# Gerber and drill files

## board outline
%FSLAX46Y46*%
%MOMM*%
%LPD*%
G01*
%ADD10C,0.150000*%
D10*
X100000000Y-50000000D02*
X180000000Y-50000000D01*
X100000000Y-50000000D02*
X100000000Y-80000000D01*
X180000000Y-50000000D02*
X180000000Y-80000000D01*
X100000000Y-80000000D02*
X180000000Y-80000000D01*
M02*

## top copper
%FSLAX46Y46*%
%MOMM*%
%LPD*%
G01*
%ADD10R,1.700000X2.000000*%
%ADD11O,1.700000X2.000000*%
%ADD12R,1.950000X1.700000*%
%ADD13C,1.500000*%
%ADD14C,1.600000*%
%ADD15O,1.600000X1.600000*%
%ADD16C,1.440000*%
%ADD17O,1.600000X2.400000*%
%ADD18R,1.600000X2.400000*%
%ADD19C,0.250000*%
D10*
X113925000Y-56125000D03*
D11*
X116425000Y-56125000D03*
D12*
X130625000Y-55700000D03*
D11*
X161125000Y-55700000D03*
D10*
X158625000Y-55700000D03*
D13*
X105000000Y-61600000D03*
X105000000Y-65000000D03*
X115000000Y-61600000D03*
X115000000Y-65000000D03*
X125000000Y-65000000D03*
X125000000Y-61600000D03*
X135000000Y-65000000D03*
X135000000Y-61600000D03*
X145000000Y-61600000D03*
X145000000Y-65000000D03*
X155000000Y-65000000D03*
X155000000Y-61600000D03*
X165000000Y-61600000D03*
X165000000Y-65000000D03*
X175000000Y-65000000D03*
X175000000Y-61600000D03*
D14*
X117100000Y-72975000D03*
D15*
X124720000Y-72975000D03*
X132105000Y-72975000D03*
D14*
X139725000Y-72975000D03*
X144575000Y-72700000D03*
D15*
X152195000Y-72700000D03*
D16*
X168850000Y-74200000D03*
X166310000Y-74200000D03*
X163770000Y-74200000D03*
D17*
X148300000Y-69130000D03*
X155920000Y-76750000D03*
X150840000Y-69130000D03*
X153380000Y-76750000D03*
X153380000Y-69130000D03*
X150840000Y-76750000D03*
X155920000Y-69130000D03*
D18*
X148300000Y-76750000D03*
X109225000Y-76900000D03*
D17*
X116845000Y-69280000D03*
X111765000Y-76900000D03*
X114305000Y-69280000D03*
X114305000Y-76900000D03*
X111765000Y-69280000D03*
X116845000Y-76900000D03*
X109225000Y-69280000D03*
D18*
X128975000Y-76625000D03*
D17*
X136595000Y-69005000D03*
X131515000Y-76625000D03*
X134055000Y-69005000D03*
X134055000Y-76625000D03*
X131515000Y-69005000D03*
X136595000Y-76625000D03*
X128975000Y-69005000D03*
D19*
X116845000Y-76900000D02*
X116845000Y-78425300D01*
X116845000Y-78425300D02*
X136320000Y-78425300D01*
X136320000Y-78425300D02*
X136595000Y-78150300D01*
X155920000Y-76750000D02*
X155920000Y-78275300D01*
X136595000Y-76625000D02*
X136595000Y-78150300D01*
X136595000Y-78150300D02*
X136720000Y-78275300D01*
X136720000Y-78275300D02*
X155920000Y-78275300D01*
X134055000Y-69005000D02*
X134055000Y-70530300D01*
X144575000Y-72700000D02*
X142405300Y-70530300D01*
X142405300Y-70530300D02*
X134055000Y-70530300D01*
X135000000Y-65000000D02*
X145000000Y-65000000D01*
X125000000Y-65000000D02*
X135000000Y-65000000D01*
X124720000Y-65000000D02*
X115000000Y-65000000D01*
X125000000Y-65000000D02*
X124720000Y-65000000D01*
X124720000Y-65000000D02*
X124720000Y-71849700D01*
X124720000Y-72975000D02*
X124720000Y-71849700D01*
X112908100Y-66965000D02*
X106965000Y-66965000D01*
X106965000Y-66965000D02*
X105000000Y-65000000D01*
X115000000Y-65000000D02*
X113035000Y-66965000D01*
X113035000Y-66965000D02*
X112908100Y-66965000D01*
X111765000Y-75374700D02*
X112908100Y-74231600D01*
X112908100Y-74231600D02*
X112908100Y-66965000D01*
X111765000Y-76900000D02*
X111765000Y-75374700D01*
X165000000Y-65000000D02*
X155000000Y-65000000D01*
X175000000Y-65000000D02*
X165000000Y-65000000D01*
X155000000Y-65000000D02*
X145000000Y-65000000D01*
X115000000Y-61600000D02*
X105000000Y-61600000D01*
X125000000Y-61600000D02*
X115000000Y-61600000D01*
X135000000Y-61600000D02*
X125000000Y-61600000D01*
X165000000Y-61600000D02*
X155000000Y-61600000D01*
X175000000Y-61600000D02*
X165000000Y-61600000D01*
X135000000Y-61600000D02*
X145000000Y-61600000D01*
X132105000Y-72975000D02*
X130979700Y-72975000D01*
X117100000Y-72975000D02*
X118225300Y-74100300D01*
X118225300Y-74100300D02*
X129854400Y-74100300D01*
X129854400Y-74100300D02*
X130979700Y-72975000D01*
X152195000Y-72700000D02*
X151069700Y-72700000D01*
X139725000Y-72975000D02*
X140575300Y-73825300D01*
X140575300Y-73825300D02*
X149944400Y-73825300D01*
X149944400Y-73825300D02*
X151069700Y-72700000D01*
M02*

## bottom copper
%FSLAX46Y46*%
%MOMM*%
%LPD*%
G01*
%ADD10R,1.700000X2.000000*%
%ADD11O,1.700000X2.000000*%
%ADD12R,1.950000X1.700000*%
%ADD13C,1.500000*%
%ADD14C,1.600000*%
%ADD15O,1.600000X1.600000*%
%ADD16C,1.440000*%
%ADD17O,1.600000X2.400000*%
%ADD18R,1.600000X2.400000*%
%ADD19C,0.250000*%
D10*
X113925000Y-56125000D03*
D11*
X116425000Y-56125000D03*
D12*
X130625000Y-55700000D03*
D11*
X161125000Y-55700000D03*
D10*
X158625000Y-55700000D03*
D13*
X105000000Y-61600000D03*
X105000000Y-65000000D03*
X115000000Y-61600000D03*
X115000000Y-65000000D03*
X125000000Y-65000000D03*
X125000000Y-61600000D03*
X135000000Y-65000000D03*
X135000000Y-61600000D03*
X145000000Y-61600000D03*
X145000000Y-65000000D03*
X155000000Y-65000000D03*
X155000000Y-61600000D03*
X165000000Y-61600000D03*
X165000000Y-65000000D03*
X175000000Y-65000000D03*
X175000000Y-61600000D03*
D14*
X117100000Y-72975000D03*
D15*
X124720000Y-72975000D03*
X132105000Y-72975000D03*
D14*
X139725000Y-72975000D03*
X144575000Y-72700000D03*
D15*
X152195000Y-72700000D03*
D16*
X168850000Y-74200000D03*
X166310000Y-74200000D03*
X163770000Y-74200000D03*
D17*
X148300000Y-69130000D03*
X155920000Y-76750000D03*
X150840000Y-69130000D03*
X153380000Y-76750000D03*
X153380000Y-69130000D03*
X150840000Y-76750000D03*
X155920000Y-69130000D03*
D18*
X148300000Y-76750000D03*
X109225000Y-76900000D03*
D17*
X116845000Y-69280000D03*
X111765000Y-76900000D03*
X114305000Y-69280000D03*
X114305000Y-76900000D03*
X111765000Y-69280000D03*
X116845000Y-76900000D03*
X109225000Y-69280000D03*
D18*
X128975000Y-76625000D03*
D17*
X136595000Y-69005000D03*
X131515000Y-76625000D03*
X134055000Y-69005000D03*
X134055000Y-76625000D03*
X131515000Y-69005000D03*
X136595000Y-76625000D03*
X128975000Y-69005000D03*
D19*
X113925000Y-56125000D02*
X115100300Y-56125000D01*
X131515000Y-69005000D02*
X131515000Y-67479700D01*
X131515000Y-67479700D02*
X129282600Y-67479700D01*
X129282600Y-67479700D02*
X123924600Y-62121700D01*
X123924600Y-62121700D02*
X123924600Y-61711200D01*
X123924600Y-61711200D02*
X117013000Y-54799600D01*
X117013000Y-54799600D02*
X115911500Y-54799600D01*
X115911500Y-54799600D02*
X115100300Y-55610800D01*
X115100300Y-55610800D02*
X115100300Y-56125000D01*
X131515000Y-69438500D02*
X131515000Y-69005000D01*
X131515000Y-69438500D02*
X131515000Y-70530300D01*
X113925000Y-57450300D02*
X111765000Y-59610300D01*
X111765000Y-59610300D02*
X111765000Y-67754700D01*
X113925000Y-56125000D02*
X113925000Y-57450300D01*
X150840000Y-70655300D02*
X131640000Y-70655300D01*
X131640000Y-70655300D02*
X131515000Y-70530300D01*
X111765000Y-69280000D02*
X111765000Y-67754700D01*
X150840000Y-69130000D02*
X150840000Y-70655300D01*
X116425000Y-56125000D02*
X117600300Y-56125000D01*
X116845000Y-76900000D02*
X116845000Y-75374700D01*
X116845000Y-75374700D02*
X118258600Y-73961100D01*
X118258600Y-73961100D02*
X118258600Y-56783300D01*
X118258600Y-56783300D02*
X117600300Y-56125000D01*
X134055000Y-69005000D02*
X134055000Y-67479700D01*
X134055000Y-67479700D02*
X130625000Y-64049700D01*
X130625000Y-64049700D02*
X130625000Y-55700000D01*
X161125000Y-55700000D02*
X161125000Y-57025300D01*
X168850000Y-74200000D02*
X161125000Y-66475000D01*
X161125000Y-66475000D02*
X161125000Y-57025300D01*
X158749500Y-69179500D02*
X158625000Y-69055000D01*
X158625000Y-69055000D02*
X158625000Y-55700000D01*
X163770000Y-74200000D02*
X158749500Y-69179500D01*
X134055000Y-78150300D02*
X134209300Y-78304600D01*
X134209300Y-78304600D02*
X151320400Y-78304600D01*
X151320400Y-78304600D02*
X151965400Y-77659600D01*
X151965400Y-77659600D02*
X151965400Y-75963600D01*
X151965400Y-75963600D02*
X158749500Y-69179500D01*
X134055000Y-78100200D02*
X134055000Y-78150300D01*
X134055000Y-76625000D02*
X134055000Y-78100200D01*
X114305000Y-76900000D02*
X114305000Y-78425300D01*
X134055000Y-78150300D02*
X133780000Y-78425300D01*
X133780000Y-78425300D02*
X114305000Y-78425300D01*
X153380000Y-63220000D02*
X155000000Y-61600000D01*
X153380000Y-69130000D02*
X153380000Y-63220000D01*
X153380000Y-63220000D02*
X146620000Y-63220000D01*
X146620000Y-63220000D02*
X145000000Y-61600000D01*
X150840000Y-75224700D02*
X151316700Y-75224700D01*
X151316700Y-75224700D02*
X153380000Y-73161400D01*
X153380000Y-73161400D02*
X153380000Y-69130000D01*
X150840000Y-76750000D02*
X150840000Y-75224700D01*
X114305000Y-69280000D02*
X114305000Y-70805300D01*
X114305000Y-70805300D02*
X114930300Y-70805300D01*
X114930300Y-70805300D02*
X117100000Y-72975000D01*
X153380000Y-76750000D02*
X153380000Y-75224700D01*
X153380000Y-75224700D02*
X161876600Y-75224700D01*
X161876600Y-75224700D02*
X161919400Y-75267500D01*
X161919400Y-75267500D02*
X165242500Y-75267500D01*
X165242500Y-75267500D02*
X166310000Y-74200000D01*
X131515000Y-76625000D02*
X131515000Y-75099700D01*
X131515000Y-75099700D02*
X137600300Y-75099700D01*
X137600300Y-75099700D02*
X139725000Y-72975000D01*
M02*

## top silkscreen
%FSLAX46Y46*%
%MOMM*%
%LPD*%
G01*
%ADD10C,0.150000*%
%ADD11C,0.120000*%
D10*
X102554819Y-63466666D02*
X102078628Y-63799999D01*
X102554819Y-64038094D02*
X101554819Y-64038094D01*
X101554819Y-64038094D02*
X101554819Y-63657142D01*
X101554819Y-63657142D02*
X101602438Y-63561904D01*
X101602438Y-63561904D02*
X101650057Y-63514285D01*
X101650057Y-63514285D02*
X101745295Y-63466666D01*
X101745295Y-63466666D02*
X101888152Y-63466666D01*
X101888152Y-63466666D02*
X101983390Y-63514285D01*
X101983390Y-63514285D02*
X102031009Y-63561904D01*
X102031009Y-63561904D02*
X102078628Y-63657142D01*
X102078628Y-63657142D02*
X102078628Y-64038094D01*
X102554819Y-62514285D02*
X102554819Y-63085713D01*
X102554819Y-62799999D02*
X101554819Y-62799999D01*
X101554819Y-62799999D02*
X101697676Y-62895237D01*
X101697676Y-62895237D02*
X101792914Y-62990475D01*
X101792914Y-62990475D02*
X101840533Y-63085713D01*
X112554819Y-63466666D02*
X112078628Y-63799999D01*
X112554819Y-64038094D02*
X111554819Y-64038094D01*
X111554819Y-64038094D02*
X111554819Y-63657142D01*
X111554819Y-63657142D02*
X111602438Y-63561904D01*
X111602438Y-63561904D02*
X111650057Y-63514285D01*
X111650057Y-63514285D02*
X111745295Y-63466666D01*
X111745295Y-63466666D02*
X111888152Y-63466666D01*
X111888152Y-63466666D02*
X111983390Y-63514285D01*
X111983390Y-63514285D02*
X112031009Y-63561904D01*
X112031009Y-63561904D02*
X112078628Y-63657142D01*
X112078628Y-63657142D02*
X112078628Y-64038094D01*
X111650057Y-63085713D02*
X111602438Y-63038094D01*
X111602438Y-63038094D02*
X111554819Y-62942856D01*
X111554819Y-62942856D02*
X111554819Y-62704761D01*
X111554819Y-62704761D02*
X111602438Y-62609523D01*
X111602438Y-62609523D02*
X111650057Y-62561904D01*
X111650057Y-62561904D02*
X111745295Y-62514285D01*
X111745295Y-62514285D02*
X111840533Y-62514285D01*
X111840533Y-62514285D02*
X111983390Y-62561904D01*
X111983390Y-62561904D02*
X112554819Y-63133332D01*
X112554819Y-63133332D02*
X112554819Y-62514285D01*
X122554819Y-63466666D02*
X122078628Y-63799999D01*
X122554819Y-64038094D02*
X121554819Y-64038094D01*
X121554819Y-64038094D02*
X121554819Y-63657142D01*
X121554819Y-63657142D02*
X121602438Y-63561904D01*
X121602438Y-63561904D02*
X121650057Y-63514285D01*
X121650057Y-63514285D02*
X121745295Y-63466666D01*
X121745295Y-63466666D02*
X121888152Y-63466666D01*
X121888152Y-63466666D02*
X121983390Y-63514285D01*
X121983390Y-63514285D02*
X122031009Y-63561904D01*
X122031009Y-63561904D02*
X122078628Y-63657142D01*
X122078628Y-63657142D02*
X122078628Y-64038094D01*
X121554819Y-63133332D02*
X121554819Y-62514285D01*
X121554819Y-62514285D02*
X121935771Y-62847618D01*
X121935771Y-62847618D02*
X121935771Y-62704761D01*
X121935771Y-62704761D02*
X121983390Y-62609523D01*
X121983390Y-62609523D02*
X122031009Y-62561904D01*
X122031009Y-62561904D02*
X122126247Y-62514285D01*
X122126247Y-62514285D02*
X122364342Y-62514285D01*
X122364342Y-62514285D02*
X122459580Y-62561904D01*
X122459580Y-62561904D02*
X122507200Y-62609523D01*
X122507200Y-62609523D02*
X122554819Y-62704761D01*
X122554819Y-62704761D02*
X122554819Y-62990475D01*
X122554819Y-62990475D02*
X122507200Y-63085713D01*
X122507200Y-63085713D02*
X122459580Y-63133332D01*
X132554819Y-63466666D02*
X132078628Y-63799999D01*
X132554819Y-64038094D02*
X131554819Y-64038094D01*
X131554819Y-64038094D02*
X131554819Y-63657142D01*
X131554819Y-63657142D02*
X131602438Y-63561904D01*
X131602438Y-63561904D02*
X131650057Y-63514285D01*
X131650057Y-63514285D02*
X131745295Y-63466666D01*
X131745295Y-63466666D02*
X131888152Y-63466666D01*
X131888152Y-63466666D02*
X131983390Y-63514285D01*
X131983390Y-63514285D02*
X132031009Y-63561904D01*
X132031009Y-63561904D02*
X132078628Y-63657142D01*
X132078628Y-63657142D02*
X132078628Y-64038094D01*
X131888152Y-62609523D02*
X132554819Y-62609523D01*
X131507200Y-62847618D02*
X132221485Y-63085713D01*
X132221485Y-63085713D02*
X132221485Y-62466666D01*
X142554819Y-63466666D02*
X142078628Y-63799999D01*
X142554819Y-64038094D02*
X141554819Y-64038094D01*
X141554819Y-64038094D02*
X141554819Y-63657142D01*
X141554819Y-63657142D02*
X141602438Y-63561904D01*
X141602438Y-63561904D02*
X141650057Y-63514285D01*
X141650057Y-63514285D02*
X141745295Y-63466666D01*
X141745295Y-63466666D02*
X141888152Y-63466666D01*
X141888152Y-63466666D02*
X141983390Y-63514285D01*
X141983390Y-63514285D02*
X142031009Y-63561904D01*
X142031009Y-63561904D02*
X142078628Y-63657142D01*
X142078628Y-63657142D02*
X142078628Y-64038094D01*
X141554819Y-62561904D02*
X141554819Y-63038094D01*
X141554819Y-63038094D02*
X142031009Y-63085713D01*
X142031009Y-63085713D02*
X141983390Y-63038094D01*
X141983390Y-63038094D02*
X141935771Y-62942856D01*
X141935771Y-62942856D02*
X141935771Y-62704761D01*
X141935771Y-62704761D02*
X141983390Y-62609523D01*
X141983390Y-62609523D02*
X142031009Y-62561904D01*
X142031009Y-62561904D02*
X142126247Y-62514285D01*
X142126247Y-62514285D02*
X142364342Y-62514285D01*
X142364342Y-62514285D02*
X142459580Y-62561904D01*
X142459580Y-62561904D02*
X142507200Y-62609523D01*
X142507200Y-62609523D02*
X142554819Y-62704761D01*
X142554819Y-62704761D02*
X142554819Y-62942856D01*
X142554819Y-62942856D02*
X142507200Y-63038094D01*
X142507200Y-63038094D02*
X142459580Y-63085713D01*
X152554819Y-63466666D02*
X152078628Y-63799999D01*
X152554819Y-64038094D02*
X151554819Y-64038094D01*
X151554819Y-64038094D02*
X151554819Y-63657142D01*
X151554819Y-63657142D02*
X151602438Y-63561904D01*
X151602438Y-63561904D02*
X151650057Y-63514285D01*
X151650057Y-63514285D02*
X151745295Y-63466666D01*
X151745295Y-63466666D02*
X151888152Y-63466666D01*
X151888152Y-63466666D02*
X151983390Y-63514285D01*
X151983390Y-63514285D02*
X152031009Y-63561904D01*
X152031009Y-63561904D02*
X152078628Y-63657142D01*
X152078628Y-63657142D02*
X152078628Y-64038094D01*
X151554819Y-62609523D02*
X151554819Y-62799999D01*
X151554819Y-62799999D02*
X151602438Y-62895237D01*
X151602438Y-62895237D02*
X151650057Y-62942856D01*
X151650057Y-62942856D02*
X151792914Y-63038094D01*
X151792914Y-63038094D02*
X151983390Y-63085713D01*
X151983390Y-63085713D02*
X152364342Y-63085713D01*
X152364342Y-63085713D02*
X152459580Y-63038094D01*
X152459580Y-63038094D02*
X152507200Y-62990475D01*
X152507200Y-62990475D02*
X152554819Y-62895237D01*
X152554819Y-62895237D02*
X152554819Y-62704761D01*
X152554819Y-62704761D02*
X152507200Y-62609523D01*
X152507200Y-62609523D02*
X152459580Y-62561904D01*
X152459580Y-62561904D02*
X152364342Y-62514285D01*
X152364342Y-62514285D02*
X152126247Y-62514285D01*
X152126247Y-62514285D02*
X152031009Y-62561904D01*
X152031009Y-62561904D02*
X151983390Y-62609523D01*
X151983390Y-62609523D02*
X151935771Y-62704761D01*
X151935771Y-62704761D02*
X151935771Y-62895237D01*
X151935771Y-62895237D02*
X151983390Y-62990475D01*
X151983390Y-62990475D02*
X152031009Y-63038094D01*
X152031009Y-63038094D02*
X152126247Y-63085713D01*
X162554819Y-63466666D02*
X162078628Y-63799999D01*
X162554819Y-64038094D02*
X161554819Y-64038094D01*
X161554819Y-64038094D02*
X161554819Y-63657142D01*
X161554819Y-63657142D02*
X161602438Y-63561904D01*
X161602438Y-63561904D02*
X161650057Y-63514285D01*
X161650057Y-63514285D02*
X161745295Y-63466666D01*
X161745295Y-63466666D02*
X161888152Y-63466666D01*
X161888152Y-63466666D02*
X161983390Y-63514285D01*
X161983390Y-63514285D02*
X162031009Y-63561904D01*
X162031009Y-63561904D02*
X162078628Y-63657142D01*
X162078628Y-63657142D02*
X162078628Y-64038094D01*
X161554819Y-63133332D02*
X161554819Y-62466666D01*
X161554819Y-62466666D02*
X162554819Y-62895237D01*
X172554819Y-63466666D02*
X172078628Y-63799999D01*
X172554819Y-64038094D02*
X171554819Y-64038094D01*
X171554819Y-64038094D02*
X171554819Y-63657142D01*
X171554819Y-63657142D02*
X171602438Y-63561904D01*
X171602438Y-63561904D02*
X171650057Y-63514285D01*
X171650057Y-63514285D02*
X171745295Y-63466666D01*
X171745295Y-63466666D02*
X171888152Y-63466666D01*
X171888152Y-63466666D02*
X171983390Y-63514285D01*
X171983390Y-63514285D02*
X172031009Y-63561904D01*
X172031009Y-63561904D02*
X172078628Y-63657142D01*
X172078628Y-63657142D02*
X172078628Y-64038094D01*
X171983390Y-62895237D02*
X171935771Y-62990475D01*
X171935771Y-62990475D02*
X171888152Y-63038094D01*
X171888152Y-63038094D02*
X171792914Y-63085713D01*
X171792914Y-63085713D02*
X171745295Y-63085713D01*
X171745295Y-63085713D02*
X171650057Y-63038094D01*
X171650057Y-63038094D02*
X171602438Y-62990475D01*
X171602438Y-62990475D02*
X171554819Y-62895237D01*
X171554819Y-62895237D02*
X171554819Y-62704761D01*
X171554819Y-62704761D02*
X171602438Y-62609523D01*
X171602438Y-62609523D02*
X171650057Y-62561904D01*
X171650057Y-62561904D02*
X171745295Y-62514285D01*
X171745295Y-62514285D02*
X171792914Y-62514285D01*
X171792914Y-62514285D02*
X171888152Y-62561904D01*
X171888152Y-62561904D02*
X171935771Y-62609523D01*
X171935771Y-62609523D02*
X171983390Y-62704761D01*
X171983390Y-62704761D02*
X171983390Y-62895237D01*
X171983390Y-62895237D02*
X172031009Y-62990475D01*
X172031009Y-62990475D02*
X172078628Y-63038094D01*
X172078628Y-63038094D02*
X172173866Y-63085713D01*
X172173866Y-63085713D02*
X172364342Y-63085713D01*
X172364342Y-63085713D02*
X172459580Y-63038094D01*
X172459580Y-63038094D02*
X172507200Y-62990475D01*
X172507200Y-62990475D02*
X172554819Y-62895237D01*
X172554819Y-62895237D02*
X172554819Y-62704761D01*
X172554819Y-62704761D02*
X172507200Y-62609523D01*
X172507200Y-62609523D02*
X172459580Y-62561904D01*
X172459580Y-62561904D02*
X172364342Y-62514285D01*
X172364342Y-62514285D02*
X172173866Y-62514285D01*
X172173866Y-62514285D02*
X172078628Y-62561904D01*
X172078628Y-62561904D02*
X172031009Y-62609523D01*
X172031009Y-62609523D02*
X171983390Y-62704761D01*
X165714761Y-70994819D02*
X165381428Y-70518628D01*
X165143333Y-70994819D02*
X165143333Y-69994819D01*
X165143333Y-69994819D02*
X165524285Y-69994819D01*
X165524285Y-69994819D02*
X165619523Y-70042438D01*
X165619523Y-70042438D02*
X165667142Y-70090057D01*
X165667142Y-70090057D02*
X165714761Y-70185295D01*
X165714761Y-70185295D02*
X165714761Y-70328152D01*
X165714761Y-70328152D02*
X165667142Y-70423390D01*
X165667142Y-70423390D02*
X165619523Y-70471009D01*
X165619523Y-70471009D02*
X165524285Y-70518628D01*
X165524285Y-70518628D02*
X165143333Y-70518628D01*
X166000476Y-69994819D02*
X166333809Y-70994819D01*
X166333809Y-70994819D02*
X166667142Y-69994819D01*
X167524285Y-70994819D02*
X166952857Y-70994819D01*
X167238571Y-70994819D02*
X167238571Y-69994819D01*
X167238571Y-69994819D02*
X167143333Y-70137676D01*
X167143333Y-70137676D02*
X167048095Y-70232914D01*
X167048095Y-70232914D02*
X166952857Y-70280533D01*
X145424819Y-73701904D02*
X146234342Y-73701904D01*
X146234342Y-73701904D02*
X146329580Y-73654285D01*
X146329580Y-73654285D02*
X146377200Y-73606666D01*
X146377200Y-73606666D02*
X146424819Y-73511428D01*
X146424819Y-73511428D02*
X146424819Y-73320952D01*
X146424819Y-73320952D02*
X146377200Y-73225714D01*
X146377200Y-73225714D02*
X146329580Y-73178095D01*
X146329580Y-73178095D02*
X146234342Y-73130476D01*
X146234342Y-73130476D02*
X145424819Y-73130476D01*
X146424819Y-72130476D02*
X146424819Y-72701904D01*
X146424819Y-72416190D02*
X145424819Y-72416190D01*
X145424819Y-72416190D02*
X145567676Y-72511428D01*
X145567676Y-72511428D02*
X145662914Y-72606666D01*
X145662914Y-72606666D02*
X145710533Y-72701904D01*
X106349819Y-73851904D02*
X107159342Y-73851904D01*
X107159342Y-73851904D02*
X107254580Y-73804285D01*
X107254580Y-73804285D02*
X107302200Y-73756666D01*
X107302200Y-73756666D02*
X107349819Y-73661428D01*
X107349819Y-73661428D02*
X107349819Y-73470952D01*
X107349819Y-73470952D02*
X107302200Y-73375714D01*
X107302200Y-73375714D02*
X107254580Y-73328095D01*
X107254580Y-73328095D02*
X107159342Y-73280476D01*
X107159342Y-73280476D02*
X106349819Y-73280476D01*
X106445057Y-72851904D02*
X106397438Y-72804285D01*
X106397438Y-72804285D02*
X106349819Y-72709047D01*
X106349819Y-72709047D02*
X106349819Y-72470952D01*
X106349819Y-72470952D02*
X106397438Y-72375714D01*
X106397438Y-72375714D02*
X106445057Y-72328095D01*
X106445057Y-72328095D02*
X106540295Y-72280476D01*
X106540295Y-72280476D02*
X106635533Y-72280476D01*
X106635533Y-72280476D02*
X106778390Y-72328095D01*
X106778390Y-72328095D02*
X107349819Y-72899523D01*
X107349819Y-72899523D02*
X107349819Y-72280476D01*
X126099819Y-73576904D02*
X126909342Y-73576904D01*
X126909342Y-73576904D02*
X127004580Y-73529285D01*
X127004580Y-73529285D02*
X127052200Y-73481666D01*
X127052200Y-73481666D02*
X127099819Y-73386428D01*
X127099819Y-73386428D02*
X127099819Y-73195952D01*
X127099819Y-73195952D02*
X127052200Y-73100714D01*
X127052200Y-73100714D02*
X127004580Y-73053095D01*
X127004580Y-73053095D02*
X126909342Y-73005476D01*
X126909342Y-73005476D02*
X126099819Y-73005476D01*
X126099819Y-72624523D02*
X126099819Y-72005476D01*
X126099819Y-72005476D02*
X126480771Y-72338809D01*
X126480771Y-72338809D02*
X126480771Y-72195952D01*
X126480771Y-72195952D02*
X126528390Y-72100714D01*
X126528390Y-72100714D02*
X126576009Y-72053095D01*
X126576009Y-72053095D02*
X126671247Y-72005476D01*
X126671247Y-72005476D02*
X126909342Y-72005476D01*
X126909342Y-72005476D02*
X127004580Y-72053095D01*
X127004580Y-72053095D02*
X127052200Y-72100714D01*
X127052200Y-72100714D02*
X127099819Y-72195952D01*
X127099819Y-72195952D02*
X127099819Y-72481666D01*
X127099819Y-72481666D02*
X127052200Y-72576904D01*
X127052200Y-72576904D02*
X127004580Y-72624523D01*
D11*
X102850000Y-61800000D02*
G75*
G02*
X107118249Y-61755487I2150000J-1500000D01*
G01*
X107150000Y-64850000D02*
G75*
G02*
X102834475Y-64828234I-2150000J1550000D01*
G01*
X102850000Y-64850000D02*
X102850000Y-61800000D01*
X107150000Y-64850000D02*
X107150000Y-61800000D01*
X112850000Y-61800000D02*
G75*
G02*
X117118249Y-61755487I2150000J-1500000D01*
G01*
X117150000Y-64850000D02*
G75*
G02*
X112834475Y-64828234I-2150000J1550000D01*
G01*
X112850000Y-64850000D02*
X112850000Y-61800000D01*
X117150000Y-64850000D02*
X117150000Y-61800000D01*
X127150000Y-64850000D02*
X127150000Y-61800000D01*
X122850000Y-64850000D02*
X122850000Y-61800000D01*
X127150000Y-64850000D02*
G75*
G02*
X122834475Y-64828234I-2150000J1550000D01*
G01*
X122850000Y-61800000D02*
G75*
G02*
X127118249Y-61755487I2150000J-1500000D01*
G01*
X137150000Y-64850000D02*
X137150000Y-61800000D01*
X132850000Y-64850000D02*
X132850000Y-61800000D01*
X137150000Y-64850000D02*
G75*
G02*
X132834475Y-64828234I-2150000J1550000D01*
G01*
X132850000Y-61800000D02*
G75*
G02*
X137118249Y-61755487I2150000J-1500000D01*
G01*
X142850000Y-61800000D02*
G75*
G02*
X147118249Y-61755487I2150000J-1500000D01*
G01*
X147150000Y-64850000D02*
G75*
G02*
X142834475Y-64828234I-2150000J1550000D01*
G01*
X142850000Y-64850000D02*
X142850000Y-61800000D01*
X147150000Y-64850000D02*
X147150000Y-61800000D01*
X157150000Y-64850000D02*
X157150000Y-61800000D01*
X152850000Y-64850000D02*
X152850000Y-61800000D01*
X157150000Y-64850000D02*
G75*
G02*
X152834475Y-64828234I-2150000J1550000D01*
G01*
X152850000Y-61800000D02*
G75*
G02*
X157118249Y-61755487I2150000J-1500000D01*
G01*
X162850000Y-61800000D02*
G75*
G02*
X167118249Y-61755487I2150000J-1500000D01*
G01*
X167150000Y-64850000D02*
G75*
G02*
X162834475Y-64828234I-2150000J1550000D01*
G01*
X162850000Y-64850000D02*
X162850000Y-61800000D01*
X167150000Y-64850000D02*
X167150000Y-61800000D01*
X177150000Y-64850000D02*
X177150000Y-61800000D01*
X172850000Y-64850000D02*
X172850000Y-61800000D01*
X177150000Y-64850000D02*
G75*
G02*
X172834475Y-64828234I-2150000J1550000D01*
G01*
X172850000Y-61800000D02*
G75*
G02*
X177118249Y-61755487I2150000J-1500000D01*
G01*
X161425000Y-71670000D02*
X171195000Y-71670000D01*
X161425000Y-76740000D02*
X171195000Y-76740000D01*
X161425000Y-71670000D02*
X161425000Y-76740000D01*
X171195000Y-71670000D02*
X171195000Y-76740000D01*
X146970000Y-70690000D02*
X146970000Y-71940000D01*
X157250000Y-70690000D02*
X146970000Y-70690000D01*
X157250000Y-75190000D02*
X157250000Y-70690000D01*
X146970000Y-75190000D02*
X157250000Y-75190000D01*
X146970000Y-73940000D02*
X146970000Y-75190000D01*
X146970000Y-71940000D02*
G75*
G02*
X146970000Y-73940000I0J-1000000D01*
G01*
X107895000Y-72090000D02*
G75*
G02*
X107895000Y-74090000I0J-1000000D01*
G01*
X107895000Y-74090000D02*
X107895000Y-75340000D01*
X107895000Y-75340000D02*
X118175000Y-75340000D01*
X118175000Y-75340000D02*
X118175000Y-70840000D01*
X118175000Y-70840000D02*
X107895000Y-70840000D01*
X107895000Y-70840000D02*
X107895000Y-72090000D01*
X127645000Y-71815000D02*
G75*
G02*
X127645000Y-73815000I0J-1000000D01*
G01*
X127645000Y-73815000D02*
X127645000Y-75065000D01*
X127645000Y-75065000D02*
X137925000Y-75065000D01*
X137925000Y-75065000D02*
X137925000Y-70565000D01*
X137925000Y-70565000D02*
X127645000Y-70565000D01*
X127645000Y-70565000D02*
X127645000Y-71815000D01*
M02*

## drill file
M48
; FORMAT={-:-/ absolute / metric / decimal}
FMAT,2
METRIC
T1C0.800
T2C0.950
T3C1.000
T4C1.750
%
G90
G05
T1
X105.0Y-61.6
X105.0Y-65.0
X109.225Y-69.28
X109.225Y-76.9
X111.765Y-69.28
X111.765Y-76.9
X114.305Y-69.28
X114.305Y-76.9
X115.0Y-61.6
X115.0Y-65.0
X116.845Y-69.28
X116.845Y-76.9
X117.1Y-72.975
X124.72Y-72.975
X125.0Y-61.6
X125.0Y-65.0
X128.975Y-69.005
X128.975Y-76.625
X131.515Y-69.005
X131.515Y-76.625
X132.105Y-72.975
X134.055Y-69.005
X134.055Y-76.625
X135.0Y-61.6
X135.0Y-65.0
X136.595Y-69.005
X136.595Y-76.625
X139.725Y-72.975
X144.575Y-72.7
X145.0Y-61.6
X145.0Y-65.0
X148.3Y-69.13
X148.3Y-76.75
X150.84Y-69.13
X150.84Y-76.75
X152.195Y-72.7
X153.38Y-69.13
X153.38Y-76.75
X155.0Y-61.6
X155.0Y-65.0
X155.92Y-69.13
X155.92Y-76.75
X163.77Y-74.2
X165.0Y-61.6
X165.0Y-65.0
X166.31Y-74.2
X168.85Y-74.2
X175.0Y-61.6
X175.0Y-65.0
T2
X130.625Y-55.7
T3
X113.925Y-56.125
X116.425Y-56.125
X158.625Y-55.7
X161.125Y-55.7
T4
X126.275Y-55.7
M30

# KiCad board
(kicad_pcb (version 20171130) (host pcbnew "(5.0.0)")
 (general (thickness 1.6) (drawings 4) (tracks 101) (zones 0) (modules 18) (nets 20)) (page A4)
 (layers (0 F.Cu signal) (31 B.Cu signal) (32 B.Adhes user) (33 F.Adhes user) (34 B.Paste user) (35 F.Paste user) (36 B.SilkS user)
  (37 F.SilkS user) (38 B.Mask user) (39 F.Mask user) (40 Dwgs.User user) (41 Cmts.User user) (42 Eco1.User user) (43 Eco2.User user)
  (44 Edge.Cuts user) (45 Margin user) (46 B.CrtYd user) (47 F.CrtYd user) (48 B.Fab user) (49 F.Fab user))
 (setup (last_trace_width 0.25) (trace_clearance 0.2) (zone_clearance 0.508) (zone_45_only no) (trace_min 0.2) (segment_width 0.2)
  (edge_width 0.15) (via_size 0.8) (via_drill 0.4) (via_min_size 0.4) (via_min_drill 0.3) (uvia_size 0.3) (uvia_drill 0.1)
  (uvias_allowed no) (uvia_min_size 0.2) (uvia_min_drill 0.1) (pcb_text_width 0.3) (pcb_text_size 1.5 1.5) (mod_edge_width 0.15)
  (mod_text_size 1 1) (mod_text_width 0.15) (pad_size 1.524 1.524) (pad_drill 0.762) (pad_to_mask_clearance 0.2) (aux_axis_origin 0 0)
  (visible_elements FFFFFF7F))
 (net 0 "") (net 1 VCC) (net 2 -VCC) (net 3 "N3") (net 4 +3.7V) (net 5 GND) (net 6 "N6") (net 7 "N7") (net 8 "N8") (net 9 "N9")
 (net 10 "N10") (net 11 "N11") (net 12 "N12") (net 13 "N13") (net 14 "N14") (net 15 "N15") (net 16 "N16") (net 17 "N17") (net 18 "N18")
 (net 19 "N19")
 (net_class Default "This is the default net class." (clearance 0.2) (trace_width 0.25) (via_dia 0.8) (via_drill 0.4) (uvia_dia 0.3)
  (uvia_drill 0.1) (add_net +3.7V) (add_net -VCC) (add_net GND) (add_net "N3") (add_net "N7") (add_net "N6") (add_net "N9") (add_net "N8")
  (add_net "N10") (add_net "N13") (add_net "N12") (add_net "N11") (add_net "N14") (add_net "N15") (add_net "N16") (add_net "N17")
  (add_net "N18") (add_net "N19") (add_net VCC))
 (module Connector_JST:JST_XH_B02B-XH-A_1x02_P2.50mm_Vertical (layer B.Cu) (at 113.925 56.125)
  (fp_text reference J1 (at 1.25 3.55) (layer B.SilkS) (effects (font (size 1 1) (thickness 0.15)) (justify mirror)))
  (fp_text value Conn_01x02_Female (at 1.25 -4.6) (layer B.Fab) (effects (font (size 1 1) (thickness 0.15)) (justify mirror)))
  (pad 1 thru_hole rect (at 0 0) (size 1.7 2) (drill 1) (layers *.Cu *.Mask) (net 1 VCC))
  (pad 2 thru_hole oval (at 2.5 0) (size 1.7 2) (drill 1) (layers *.Cu *.Mask) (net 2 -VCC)))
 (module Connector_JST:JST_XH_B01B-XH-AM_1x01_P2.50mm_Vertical (layer B.Cu) (at 130.625 55.7 90)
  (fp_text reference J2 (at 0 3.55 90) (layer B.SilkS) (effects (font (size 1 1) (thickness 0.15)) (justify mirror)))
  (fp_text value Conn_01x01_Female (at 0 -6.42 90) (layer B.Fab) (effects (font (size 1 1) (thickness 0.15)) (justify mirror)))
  (pad 1 thru_hole rect (at 0 0 90) (size 1.7 1.95) (drill 0.95) (layers *.Cu *.Mask) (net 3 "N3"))
  (pad "" np_thru_hole circle (at 0 -4.35 90) (size 1.75 1.75) (drill 1.75) (layers *.Cu *.Mask)))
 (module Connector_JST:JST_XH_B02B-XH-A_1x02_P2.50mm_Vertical (layer B.Cu) (at 158.625 55.7)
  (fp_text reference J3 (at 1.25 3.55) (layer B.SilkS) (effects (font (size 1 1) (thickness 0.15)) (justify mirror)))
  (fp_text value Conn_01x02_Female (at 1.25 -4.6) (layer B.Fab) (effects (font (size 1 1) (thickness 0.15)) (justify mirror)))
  (pad 2 thru_hole oval (at 2.5 0) (size 1.7 2) (drill 1) (layers *.Cu *.Mask) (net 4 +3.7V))
  (pad 1 thru_hole rect (at 0 0) (size 1.7 2) (drill 1) (layers *.Cu *.Mask) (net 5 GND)))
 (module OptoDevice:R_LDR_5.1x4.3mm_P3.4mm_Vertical (layer F.Cu) (at 105 65 90)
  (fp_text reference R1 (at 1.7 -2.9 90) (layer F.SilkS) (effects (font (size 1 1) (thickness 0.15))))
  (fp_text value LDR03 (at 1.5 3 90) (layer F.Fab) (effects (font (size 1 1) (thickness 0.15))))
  (fp_arc (start 1.7 0) (end 3.2 -2.15) (angle 109) (layer F.SilkS) (width 0.12))
  (fp_arc (start 1.7 0) (end 0.15 2.15) (angle 109) (layer F.SilkS) (width 0.12))
  (fp_line (start 0.15 -2.15) (end 3.2 -2.15) (layer F.SilkS) (width 0.12))
  (fp_line (start 0.15 2.15) (end 3.2 2.15) (layer F.SilkS) (width 0.12))
  (pad 2 thru_hole circle (at 3.4 0 90) (size 1.5 1.5) (drill 0.8) (layers *.Cu *.Mask) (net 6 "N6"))
  (pad 1 thru_hole circle (at 0 0 90) (size 1.5 1.5) (drill 0.8) (layers *.Cu *.Mask) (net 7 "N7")))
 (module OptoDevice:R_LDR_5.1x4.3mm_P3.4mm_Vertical (layer F.Cu) (at 115 65 90)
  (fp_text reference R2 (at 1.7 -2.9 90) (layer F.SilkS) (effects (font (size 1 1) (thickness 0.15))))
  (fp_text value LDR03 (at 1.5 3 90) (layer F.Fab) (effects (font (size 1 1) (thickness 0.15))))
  (fp_arc (start 1.7 0) (end 3.2 -2.15) (angle 109) (layer F.SilkS) (width 0.12))
  (fp_arc (start 1.7 0) (end 0.15 2.15) (angle 109) (layer F.SilkS) (width 0.12))
  (fp_line (start 0.15 -2.15) (end 3.2 -2.15) (layer F.SilkS) (width 0.12))
  (fp_line (start 0.15 2.15) (end 3.2 2.15) (layer F.SilkS) (width 0.12))
  (pad 2 thru_hole circle (at 3.4 0 90) (size 1.5 1.5) (drill 0.8) (layers *.Cu *.Mask) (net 6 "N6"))
  (pad 1 thru_hole circle (at 0 0 90) (size 1.5 1.5) (drill 0.8) (layers *.Cu *.Mask) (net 7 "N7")))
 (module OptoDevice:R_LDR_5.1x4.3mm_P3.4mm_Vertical (layer F.Cu) (at 125 65 90)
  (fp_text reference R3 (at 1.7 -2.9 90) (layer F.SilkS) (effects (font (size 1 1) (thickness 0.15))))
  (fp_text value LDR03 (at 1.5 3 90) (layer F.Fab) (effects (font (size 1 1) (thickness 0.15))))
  (fp_line (start 0.15 2.15) (end 3.2 2.15) (layer F.SilkS) (width 0.12))
  (fp_line (start 0.15 -2.15) (end 3.2 -2.15) (layer F.SilkS) (width 0.12))
  (fp_arc (start 1.7 0) (end 0.15 2.15) (angle 109) (layer F.SilkS) (width 0.12))
  (fp_arc (start 1.7 0) (end 3.2 -2.15) (angle 109) (layer F.SilkS) (width 0.12))
  (pad 1 thru_hole circle (at 0 0 90) (size 1.5 1.5) (drill 0.8) (layers *.Cu *.Mask) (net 7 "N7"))
  (pad 2 thru_hole circle (at 3.4 0 90) (size 1.5 1.5) (drill 0.8) (layers *.Cu *.Mask) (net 6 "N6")))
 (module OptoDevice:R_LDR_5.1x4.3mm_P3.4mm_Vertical (layer F.Cu) (at 135 65 90)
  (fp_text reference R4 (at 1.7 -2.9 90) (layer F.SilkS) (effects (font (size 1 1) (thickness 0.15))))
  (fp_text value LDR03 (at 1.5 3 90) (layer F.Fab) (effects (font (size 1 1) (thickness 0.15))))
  (fp_line (start 0.15 2.15) (end 3.2 2.15) (layer F.SilkS) (width 0.12))
  (fp_line (start 0.15 -2.15) (end 3.2 -2.15) (layer F.SilkS) (width 0.12))
  (fp_arc (start 1.7 0) (end 0.15 2.15) (angle 109) (layer F.SilkS) (width 0.12))
  (fp_arc (start 1.7 0) (end 3.2 -2.15) (angle 109) (layer F.SilkS) (width 0.12))
  (pad 1 thru_hole circle (at 0 0 90) (size 1.5 1.5) (drill 0.8) (layers *.Cu *.Mask) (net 7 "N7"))
  (pad 2 thru_hole circle (at 3.4 0 90) (size 1.5 1.5) (drill 0.8) (layers *.Cu *.Mask) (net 6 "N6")))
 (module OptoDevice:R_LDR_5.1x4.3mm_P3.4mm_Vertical (layer F.Cu) (at 145 65 90)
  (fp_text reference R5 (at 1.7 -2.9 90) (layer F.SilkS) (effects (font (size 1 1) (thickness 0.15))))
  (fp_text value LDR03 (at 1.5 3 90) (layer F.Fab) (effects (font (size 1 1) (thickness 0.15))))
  (fp_arc (start 1.7 0) (end 3.2 -2.15) (angle 109) (layer F.SilkS) (width 0.12))
  (fp_arc (start 1.7 0) (end 0.15 2.15) (angle 109) (layer F.SilkS) (width 0.12))
  (fp_line (start 0.15 -2.15) (end 3.2 -2.15) (layer F.SilkS) (width 0.12))
  (fp_line (start 0.15 2.15) (end 3.2 2.15) (layer F.SilkS) (width 0.12))
  (pad 2 thru_hole circle (at 3.4 0 90) (size 1.5 1.5) (drill 0.8) (layers *.Cu *.Mask) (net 6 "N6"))
  (pad 1 thru_hole circle (at 0 0 90) (size 1.5 1.5) (drill 0.8) (layers *.Cu *.Mask) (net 7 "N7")))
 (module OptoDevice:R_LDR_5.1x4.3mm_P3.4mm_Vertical (layer F.Cu) (at 155 65 90)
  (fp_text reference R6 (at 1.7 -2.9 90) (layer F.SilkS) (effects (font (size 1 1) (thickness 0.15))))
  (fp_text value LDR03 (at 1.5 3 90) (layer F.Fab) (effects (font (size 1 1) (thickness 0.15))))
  (fp_line (start 0.15 2.15) (end 3.2 2.15) (layer F.SilkS) (width 0.12))
  (fp_line (start 0.15 -2.15) (end 3.2 -2.15) (layer F.SilkS) (width 0.12))
  (fp_arc (start 1.7 0) (end 0.15 2.15) (angle 109) (layer F.SilkS) (width 0.12))
  (fp_arc (start 1.7 0) (end 3.2 -2.15) (angle 109) (layer F.SilkS) (width 0.12))
  (pad 1 thru_hole circle (at 0 0 90) (size 1.5 1.5) (drill 0.8) (layers *.Cu *.Mask) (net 7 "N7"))
  (pad 2 thru_hole circle (at 3.4 0 90) (size 1.5 1.5) (drill 0.8) (layers *.Cu *.Mask) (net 6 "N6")))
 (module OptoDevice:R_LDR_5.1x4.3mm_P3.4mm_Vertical (layer F.Cu) (at 165 65 90)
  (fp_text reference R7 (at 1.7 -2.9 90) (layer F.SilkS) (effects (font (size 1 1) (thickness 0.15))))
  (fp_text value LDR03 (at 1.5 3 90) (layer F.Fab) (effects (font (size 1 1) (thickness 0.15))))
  (fp_arc (start 1.7 0) (end 3.2 -2.15) (angle 109) (layer F.SilkS) (width 0.12))
  (fp_arc (start 1.7 0) (end 0.15 2.15) (angle 109) (layer F.SilkS) (width 0.12))
  (fp_line (start 0.15 -2.15) (end 3.2 -2.15) (layer F.SilkS) (width 0.12))
  (fp_line (start 0.15 2.15) (end 3.2 2.15) (layer F.SilkS) (width 0.12))
  (pad 2 thru_hole circle (at 3.4 0 90) (size 1.5 1.5) (drill 0.8) (layers *.Cu *.Mask) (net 6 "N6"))
  (pad 1 thru_hole circle (at 0 0 90) (size 1.5 1.5) (drill 0.8) (layers *.Cu *.Mask) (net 7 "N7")))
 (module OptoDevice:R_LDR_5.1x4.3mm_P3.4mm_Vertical (layer F.Cu) (at 175 65 90)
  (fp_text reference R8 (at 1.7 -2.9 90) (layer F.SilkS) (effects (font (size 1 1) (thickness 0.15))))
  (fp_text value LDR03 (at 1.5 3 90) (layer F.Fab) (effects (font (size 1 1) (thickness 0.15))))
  (fp_line (start 0.15 2.15) (end 3.2 2.15) (layer F.SilkS) (width 0.12))
  (fp_line (start 0.15 -2.15) (end 3.2 -2.15) (layer F.SilkS) (width 0.12))
  (fp_arc (start 1.7 0) (end 0.15 2.15) (angle 109) (layer F.SilkS) (width 0.12))
  (fp_arc (start 1.7 0) (end 3.2 -2.15) (angle 109) (layer F.SilkS) (width 0.12))
  (pad 1 thru_hole circle (at 0 0 90) (size 1.5 1.5) (drill 0.8) (layers *.Cu *.Mask) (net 7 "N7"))
  (pad 2 thru_hole circle (at 3.4 0 90) (size 1.5 1.5) (drill 0.8) (layers *.Cu *.Mask) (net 6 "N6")))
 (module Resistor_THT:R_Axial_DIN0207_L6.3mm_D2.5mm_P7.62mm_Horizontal (layer B.Cu) (at 117.1 72.975)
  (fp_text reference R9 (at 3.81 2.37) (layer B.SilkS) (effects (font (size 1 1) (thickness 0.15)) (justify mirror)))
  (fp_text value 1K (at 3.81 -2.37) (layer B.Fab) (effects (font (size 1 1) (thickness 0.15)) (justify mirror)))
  (pad 1 thru_hole circle (at 0 0) (size 1.6 1.6) (drill 0.8) (layers *.Cu *.Mask) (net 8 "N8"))
  (pad 2 thru_hole oval (at 7.62 0) (size 1.6 1.6) (drill 0.8) (layers *.Cu *.Mask) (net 7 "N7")))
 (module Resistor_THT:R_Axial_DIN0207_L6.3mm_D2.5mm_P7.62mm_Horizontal (layer B.Cu) (at 139.725 72.975 180)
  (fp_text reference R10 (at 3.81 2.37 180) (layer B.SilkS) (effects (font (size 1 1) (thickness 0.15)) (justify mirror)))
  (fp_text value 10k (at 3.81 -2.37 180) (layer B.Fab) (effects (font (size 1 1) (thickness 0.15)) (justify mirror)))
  (pad 2 thru_hole oval (at 7.62 0 180) (size 1.6 1.6) (drill 0.8) (layers *.Cu *.Mask) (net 8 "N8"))
  (pad 1 thru_hole circle (at 0 0 180) (size 1.6 1.6) (drill 0.8) (layers *.Cu *.Mask) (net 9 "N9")))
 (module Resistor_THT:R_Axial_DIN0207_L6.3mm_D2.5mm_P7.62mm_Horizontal (layer B.Cu) (at 144.575 72.7)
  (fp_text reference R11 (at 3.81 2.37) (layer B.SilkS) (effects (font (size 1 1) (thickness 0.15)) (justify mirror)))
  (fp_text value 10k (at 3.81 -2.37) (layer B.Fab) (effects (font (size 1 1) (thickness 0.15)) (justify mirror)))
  (pad 1 thru_hole circle (at 0 0) (size 1.6 1.6) (drill 0.8) (layers *.Cu *.Mask) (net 3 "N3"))
  (pad 2 thru_hole oval (at 7.62 0) (size 1.6 1.6) (drill 0.8) (layers *.Cu *.Mask) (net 9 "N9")))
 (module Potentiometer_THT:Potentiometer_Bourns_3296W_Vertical (layer F.Cu) (at 168.85 74.2)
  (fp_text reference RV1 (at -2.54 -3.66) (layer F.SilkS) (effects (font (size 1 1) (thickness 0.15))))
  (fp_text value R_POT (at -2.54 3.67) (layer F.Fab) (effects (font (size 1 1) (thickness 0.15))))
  (fp_line (start -7.425 -2.53) (end 2.345 -2.53) (layer F.SilkS) (width 0.12))
  (fp_line (start -7.425 2.54) (end 2.345 2.54) (layer F.SilkS) (width 0.12))
  (fp_line (start -7.425 -2.53) (end -7.425 2.54) (layer F.SilkS) (width 0.12))
  (fp_line (start 2.345 -2.53) (end 2.345 2.54) (layer F.SilkS) (width 0.12))
  (pad 1 thru_hole circle (at 0 0) (size 1.44 1.44) (drill 0.8) (layers *.Cu *.Mask) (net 4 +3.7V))
  (pad 2 thru_hole circle (at -2.54 0) (size 1.44 1.44) (drill 0.8) (layers *.Cu *.Mask) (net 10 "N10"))
  (pad 3 thru_hole circle (at -5.08 0) (size 1.44 1.44) (drill 0.8) (layers *.Cu *.Mask) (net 5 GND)))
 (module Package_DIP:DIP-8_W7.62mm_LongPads (layer F.Cu) (at 148.3 76.75 90)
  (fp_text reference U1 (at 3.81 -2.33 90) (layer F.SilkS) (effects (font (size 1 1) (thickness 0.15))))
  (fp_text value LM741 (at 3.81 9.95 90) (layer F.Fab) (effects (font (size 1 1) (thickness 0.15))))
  (fp_line (start 6.06 -1.33) (end 4.81 -1.33) (layer F.SilkS) (width 0.12))
  (fp_line (start 6.06 8.95) (end 6.06 -1.33) (layer F.SilkS) (width 0.12))
  (fp_line (start 1.56 8.95) (end 6.06 8.95) (layer F.SilkS) (width 0.12))
  (fp_line (start 1.56 -1.33) (end 1.56 8.95) (layer F.SilkS) (width 0.12))
  (fp_line (start 2.81 -1.33) (end 1.56 -1.33) (layer F.SilkS) (width 0.12))
  (fp_arc (start 3.81 -1.33) (end 2.81 -1.33) (angle -180) (layer F.SilkS) (width 0.12))
  (pad 8 thru_hole oval (at 7.62 0 90) (size 2.4 1.6) (drill 0.8) (layers *.Cu *.Mask) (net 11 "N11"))
  (pad 4 thru_hole oval (at 0 7.62 90) (size 2.4 1.6) (drill 0.8) (layers *.Cu *.Mask) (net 2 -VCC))
  (pad 7 thru_hole oval (at 7.62 2.54 90) (size 2.4 1.6) (drill 0.8) (layers *.Cu *.Mask) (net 1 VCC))
  (pad 3 thru_hole oval (at 0 5.08 90) (size 2.4 1.6) (drill 0.8) (layers *.Cu *.Mask) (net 10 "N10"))
  (pad 6 thru_hole oval (at 7.62 5.08 90) (size 2.4 1.6) (drill 0.8) (layers *.Cu *.Mask) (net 6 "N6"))
  (pad 2 thru_hole oval (at 0 2.54 90) (size 2.4 1.6) (drill 0.8) (layers *.Cu *.Mask) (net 6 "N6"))
  (pad 5 thru_hole oval (at 7.62 7.62 90) (size 2.4 1.6) (drill 0.8) (layers *.Cu *.Mask) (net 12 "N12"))
  (pad 1 thru_hole rect (at 0 0 90) (size 2.4 1.6) (drill 0.8) (layers *.Cu *.Mask) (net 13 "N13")))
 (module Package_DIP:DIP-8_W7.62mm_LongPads (layer F.Cu) (at 109.225 76.9 90)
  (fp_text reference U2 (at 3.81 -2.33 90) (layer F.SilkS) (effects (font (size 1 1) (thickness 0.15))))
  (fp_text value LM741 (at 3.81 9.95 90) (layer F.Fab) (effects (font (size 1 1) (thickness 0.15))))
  (fp_arc (start 3.81 -1.33) (end 2.81 -1.33) (angle -180) (layer F.SilkS) (width 0.12))
  (fp_line (start 2.81 -1.33) (end 1.56 -1.33) (layer F.SilkS) (width 0.12))
  (fp_line (start 1.56 -1.33) (end 1.56 8.95) (layer F.SilkS) (width 0.12))
  (fp_line (start 1.56 8.95) (end 6.06 8.95) (layer F.SilkS) (width 0.12))
  (fp_line (start 6.06 8.95) (end 6.06 -1.33) (layer F.SilkS) (width 0.12))
  (fp_line (start 6.06 -1.33) (end 4.81 -1.33) (layer F.SilkS) (width 0.12))
  (pad 1 thru_hole rect (at 0 0 90) (size 2.4 1.6) (drill 0.8) (layers *.Cu *.Mask) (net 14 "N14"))
  (pad 5 thru_hole oval (at 7.62 7.62 90) (size 2.4 1.6) (drill 0.8) (layers *.Cu *.Mask) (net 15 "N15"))
  (pad 2 thru_hole oval (at 0 2.54 90) (size 2.4 1.6) (drill 0.8) (layers *.Cu *.Mask) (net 7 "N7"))
  (pad 6 thru_hole oval (at 7.62 5.08 90) (size 2.4 1.6) (drill 0.8) (layers *.Cu *.Mask) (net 8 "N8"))
  (pad 3 thru_hole oval (at 0 5.08 90) (size 2.4 1.6) (drill 0.8) (layers *.Cu *.Mask) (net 5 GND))
  (pad 7 thru_hole oval (at 7.62 2.54 90) (size 2.4 1.6) (drill 0.8) (layers *.Cu *.Mask) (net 1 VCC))
  (pad 4 thru_hole oval (at 0 7.62 90) (size 2.4 1.6) (drill 0.8) (layers *.Cu *.Mask) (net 2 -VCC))
  (pad 8 thru_hole oval (at 7.62 0 90) (size 2.4 1.6) (drill 0.8) (layers *.Cu *.Mask) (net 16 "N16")))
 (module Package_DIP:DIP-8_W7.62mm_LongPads (layer F.Cu) (at 128.975 76.625 90)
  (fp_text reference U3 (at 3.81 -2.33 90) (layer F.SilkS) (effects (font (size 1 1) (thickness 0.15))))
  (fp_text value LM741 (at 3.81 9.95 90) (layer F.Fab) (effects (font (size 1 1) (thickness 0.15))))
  (fp_arc (start 3.81 -1.33) (end 2.81 -1.33) (angle -180) (layer F.SilkS) (width 0.12))
  (fp_line (start 2.81 -1.33) (end 1.56 -1.33) (layer F.SilkS) (width 0.12))
  (fp_line (start 1.56 -1.33) (end 1.56 8.95) (layer F.SilkS) (width 0.12))
  (fp_line (start 1.56 8.95) (end 6.06 8.95) (layer F.SilkS) (width 0.12))
  (fp_line (start 6.06 8.95) (end 6.06 -1.33) (layer F.SilkS) (width 0.12))
  (fp_line (start 6.06 -1.33) (end 4.81 -1.33) (layer F.SilkS) (width 0.12))
  (pad 1 thru_hole rect (at 0 0 90) (size 2.4 1.6) (drill 0.8) (layers *.Cu *.Mask) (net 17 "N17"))
  (pad 5 thru_hole oval (at 7.62 7.62 90) (size 2.4 1.6) (drill 0.8) (layers *.Cu *.Mask) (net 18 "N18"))
  (pad 2 thru_hole oval (at 0 2.54 90) (size 2.4 1.6) (drill 0.8) (layers *.Cu *.Mask) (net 9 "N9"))
  (pad 6 thru_hole oval (at 7.62 5.08 90) (size 2.4 1.6) (drill 0.8) (layers *.Cu *.Mask) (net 3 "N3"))
  (pad 3 thru_hole oval (at 0 5.08 90) (size 2.4 1.6) (drill 0.8) (layers *.Cu *.Mask) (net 5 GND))
  (pad 7 thru_hole oval (at 7.62 2.54 90) (size 2.4 1.6) (drill 0.8) (layers *.Cu *.Mask) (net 1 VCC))
  (pad 4 thru_hole oval (at 0 7.62 90) (size 2.4 1.6) (drill 0.8) (layers *.Cu *.Mask) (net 2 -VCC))
  (pad 8 thru_hole oval (at 7.62 0 90) (size 2.4 1.6) (drill 0.8) (layers *.Cu *.Mask) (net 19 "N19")))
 (gr_line (start 100 50) (end 180 50) (layer Edge.Cuts) (width 0.15))
 (gr_line (start 100 50) (end 100 80) (layer Edge.Cuts) (width 0.15))
 (gr_line (start 180 50) (end 180 80) (layer Edge.Cuts) (width 0.15))
 (gr_line (start 100 80) (end 180 80) (layer Edge.Cuts) (width 0.15))
 (segment (start 113.925 56.125) (end 115.1003 56.125) (width 0.25) (layer B.Cu) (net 1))
 (segment (start 131.515 69.005) (end 131.515 67.4797) (width 0.25) (layer B.Cu) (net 1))
 (segment (start 131.515 67.4797) (end 129.2826 67.4797) (width 0.25) (layer B.Cu) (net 1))
 (segment (start 129.2826 67.4797) (end 123.9246 62.1217) (width 0.25) (layer B.Cu) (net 1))
 (segment (start 123.9246 62.1217) (end 123.9246 61.7112) (width 0.25) (layer B.Cu) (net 1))
 (segment (start 123.9246 61.7112) (end 117.013 54.7996) (width 0.25) (layer B.Cu) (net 1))
 (segment (start 117.013 54.7996) (end 115.9115 54.7996) (width 0.25) (layer B.Cu) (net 1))
 (segment (start 115.9115 54.7996) (end 115.1003 55.6108) (width 0.25) (layer B.Cu) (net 1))
 (segment (start 115.1003 55.6108) (end 115.1003 56.125) (width 0.25) (layer B.Cu) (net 1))
 (segment (start 131.515 69.4385) (end 131.515 69.005) (width 0.25) (layer B.Cu) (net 1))
 (segment (start 131.515 69.4385) (end 131.515 70.5303) (width 0.25) (layer B.Cu) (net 1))
 (segment (start 113.925 57.4503) (end 111.765 59.6103) (width 0.25) (layer B.Cu) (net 1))
 (segment (start 111.765 59.6103) (end 111.765 67.7547) (width 0.25) (layer B.Cu) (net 1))
 (segment (start 113.925 56.125) (end 113.925 57.4503) (width 0.25) (layer B.Cu) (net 1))
 (segment (start 150.84 70.6553) (end 131.64 70.6553) (width 0.25) (layer B.Cu) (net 1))
 (segment (start 131.64 70.6553) (end 131.515 70.5303) (width 0.25) (layer B.Cu) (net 1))
 (segment (start 111.765 69.28) (end 111.765 67.7547) (width 0.25) (layer B.Cu) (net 1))
 (segment (start 150.84 69.13) (end 150.84 70.6553) (width 0.25) (layer B.Cu) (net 1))
 (segment (start 116.425 56.125) (end 117.6003 56.125) (width 0.25) (layer B.Cu) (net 2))
 (segment (start 116.845 76.9) (end 116.845 75.3747) (width 0.25) (layer B.Cu) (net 2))
 (segment (start 116.845 75.3747) (end 118.2586 73.9611) (width 0.25) (layer B.Cu) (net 2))
 (segment (start 118.2586 73.9611) (end 118.2586 56.7833) (width 0.25) (layer B.Cu) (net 2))
 (segment (start 118.2586 56.7833) (end 117.6003 56.125) (width 0.25) (layer B.Cu) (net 2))
 (segment (start 116.845 76.9) (end 116.845 78.4253) (width 0.25) (layer F.Cu) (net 2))
 (segment (start 116.845 78.4253) (end 136.32 78.4253) (width 0.25) (layer F.Cu) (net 2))
 (segment (start 136.32 78.4253) (end 136.595 78.1503) (width 0.25) (layer F.Cu) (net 2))
 (segment (start 155.92 76.75) (end 155.92 78.2753) (width 0.25) (layer F.Cu) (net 2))
 (segment (start 136.595 76.625) (end 136.595 78.1503) (width 0.25) (layer F.Cu) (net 2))
 (segment (start 136.595 78.1503) (end 136.72 78.2753) (width 0.25) (layer F.Cu) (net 2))
 (segment (start 136.72 78.2753) (end 155.92 78.2753) (width 0.25) (layer F.Cu) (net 2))
 (segment (start 134.055 69.005) (end 134.055 67.4797) (width 0.25) (layer B.Cu) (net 3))
 (segment (start 134.055 67.4797) (end 130.625 64.0497) (width 0.25) (layer B.Cu) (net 3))
 (segment (start 130.625 64.0497) (end 130.625 55.7) (width 0.25) (layer B.Cu) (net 3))
 (segment (start 134.055 69.005) (end 134.055 70.5303) (width 0.25) (layer F.Cu) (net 3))
 (segment (start 144.575 72.7) (end 142.4053 70.5303) (width 0.25) (layer F.Cu) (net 3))
 (segment (start 142.4053 70.5303) (end 134.055 70.5303) (width 0.25) (layer F.Cu) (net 3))
 (segment (start 161.125 55.7) (end 161.125 57.0253) (width 0.25) (layer B.Cu) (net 4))
 (segment (start 168.85 74.2) (end 161.125 66.475) (width 0.25) (layer B.Cu) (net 4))
 (segment (start 161.125 66.475) (end 161.125 57.0253) (width 0.25) (layer B.Cu) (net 4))
 (segment (start 158.7495 69.1795) (end 158.625 69.055) (width 0.25) (layer B.Cu) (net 5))
 (segment (start 158.625 69.055) (end 158.625 55.7) (width 0.25) (layer B.Cu) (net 5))
 (segment (start 163.77 74.2) (end 158.7495 69.1795) (width 0.25) (layer B.Cu) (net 5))
 (segment (start 134.055 78.1503) (end 134.2093 78.3046) (width 0.25) (layer B.Cu) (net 5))
 (segment (start 134.2093 78.3046) (end 151.3204 78.3046) (width 0.25) (layer B.Cu) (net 5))
 (segment (start 151.3204 78.3046) (end 151.9654 77.6596) (width 0.25) (layer B.Cu) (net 5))
 (segment (start 151.9654 77.6596) (end 151.9654 75.9636) (width 0.25) (layer B.Cu) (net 5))
 (segment (start 151.9654 75.9636) (end 158.7495 69.1795) (width 0.25) (layer B.Cu) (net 5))
 (segment (start 134.055 78.1002) (end 134.055 78.1503) (width 0.25) (layer B.Cu) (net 5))
 (segment (start 134.055 76.625) (end 134.055 78.1002) (width 0.25) (layer B.Cu) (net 5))
 (segment (start 114.305 76.9) (end 114.305 78.4253) (width 0.25) (layer B.Cu) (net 5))
 (segment (start 134.055 78.1503) (end 133.78 78.4253) (width 0.25) (layer B.Cu) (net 5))
 (segment (start 133.78 78.4253) (end 114.305 78.4253) (width 0.25) (layer B.Cu) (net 5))
 (segment (start 135 65) (end 145 65) (width 0.25) (layer F.Cu) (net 7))
 (segment (start 125 65) (end 135 65) (width 0.25) (layer F.Cu) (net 7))
 (segment (start 124.72 65) (end 115 65) (width 0.25) (layer F.Cu) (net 7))
 (segment (start 125 65) (end 124.72 65) (width 0.25) (layer F.Cu) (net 7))
 (segment (start 124.72 65) (end 124.72 71.8497) (width 0.25) (layer F.Cu) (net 7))
 (segment (start 124.72 72.975) (end 124.72 71.8497) (width 0.25) (layer F.Cu) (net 7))
 (segment (start 112.9081 66.965) (end 106.965 66.965) (width 0.25) (layer F.Cu) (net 7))
 (segment (start 106.965 66.965) (end 105 65) (width 0.25) (layer F.Cu) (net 7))
 (segment (start 115 65) (end 113.035 66.965) (width 0.25) (layer F.Cu) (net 7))
 (segment (start 113.035 66.965) (end 112.9081 66.965) (width 0.25) (layer F.Cu) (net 7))
 (segment (start 111.765 75.3747) (end 112.9081 74.2316) (width 0.25) (layer F.Cu) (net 7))
 (segment (start 112.9081 74.2316) (end 112.9081 66.965) (width 0.25) (layer F.Cu) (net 7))
 (segment (start 111.765 76.9) (end 111.765 75.3747) (width 0.25) (layer F.Cu) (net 7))
 (segment (start 165 65) (end 155 65) (width 0.25) (layer F.Cu) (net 7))
 (segment (start 175 65) (end 165 65) (width 0.25) (layer F.Cu) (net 7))
 (segment (start 155 65) (end 145 65) (width 0.25) (layer F.Cu) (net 7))
 (segment (start 153.38 63.22) (end 155 61.6) (width 0.25) (layer B.Cu) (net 6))
 (segment (start 153.38 69.13) (end 153.38 63.22) (width 0.25) (layer B.Cu) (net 6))
 (segment (start 153.38 63.22) (end 146.62 63.22) (width 0.25) (layer B.Cu) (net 6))
 (segment (start 146.62 63.22) (end 145 61.6) (width 0.25) (layer B.Cu) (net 6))
 (segment (start 150.84 75.2247) (end 151.3167 75.2247) (width 0.25) (layer B.Cu) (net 6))
 (segment (start 151.3167 75.2247) (end 153.38 73.1614) (width 0.25) (layer B.Cu) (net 6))
 (segment (start 153.38 73.1614) (end 153.38 69.13) (width 0.25) (layer B.Cu) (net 6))
 (segment (start 150.84 76.75) (end 150.84 75.2247) (width 0.25) (layer B.Cu) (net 6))
 (segment (start 115 61.6) (end 105 61.6) (width 0.25) (layer F.Cu) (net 6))
 (segment (start 125 61.6) (end 115 61.6) (width 0.25) (layer F.Cu) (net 6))
 (segment (start 135 61.6) (end 125 61.6) (width 0.25) (layer F.Cu) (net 6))
 (segment (start 165 61.6) (end 155 61.6) (width 0.25) (layer F.Cu) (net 6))
 (segment (start 175 61.6) (end 165 61.6) (width 0.25) (layer F.Cu) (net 6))
 (segment (start 135 61.6) (end 145 61.6) (width 0.25) (layer F.Cu) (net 6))
 (segment (start 114.305 69.28) (end 114.305 70.8053) (width 0.25) (layer B.Cu) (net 8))
 (segment (start 114.305 70.8053) (end 114.9303 70.8053) (width 0.25) (layer B.Cu) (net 8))
 (segment (start 114.9303 70.8053) (end 117.1 72.975) (width 0.25) (layer B.Cu) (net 8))
 (segment (start 132.105 72.975) (end 130.9797 72.975) (width 0.25) (layer F.Cu) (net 8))
 (segment (start 117.1 72.975) (end 118.2253 74.1003) (width 0.25) (layer F.Cu) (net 8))
 (segment (start 118.2253 74.1003) (end 129.8544 74.1003) (width 0.25) (layer F.Cu) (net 8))
 (segment (start 129.8544 74.1003) (end 130.9797 72.975) (width 0.25) (layer F.Cu) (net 8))
 (segment (start 153.38 76.75) (end 153.38 75.2247) (width 0.25) (layer B.Cu) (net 10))
 (segment (start 153.38 75.2247) (end 161.8766 75.2247) (width 0.25) (layer B.Cu) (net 10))
 (segment (start 161.8766 75.2247) (end 161.9194 75.2675) (width 0.25) (layer B.Cu) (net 10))
 (segment (start 161.9194 75.2675) (end 165.2425 75.2675) (width 0.25) (layer B.Cu) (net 10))
 (segment (start 165.2425 75.2675) (end 166.31 74.2) (width 0.25) (layer B.Cu) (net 10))
 (segment (start 152.195 72.7) (end 151.0697 72.7) (width 0.25) (layer F.Cu) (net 9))
 (segment (start 139.725 72.975) (end 140.5753 73.8253) (width 0.25) (layer F.Cu) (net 9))
 (segment (start 140.5753 73.8253) (end 149.9444 73.8253) (width 0.25) (layer F.Cu) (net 9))
 (segment (start 149.9444 73.8253) (end 151.0697 72.7) (width 0.25) (layer F.Cu) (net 9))
 (segment (start 131.515 76.625) (end 131.515 75.0997) (width 0.25) (layer B.Cu) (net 9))
 (segment (start 131.515 75.0997) (end 137.6003 75.0997) (width 0.25) (layer B.Cu) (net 9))
 (segment (start 137.6003 75.0997) (end 139.725 72.975) (width 0.25) (layer B.Cu) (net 9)))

